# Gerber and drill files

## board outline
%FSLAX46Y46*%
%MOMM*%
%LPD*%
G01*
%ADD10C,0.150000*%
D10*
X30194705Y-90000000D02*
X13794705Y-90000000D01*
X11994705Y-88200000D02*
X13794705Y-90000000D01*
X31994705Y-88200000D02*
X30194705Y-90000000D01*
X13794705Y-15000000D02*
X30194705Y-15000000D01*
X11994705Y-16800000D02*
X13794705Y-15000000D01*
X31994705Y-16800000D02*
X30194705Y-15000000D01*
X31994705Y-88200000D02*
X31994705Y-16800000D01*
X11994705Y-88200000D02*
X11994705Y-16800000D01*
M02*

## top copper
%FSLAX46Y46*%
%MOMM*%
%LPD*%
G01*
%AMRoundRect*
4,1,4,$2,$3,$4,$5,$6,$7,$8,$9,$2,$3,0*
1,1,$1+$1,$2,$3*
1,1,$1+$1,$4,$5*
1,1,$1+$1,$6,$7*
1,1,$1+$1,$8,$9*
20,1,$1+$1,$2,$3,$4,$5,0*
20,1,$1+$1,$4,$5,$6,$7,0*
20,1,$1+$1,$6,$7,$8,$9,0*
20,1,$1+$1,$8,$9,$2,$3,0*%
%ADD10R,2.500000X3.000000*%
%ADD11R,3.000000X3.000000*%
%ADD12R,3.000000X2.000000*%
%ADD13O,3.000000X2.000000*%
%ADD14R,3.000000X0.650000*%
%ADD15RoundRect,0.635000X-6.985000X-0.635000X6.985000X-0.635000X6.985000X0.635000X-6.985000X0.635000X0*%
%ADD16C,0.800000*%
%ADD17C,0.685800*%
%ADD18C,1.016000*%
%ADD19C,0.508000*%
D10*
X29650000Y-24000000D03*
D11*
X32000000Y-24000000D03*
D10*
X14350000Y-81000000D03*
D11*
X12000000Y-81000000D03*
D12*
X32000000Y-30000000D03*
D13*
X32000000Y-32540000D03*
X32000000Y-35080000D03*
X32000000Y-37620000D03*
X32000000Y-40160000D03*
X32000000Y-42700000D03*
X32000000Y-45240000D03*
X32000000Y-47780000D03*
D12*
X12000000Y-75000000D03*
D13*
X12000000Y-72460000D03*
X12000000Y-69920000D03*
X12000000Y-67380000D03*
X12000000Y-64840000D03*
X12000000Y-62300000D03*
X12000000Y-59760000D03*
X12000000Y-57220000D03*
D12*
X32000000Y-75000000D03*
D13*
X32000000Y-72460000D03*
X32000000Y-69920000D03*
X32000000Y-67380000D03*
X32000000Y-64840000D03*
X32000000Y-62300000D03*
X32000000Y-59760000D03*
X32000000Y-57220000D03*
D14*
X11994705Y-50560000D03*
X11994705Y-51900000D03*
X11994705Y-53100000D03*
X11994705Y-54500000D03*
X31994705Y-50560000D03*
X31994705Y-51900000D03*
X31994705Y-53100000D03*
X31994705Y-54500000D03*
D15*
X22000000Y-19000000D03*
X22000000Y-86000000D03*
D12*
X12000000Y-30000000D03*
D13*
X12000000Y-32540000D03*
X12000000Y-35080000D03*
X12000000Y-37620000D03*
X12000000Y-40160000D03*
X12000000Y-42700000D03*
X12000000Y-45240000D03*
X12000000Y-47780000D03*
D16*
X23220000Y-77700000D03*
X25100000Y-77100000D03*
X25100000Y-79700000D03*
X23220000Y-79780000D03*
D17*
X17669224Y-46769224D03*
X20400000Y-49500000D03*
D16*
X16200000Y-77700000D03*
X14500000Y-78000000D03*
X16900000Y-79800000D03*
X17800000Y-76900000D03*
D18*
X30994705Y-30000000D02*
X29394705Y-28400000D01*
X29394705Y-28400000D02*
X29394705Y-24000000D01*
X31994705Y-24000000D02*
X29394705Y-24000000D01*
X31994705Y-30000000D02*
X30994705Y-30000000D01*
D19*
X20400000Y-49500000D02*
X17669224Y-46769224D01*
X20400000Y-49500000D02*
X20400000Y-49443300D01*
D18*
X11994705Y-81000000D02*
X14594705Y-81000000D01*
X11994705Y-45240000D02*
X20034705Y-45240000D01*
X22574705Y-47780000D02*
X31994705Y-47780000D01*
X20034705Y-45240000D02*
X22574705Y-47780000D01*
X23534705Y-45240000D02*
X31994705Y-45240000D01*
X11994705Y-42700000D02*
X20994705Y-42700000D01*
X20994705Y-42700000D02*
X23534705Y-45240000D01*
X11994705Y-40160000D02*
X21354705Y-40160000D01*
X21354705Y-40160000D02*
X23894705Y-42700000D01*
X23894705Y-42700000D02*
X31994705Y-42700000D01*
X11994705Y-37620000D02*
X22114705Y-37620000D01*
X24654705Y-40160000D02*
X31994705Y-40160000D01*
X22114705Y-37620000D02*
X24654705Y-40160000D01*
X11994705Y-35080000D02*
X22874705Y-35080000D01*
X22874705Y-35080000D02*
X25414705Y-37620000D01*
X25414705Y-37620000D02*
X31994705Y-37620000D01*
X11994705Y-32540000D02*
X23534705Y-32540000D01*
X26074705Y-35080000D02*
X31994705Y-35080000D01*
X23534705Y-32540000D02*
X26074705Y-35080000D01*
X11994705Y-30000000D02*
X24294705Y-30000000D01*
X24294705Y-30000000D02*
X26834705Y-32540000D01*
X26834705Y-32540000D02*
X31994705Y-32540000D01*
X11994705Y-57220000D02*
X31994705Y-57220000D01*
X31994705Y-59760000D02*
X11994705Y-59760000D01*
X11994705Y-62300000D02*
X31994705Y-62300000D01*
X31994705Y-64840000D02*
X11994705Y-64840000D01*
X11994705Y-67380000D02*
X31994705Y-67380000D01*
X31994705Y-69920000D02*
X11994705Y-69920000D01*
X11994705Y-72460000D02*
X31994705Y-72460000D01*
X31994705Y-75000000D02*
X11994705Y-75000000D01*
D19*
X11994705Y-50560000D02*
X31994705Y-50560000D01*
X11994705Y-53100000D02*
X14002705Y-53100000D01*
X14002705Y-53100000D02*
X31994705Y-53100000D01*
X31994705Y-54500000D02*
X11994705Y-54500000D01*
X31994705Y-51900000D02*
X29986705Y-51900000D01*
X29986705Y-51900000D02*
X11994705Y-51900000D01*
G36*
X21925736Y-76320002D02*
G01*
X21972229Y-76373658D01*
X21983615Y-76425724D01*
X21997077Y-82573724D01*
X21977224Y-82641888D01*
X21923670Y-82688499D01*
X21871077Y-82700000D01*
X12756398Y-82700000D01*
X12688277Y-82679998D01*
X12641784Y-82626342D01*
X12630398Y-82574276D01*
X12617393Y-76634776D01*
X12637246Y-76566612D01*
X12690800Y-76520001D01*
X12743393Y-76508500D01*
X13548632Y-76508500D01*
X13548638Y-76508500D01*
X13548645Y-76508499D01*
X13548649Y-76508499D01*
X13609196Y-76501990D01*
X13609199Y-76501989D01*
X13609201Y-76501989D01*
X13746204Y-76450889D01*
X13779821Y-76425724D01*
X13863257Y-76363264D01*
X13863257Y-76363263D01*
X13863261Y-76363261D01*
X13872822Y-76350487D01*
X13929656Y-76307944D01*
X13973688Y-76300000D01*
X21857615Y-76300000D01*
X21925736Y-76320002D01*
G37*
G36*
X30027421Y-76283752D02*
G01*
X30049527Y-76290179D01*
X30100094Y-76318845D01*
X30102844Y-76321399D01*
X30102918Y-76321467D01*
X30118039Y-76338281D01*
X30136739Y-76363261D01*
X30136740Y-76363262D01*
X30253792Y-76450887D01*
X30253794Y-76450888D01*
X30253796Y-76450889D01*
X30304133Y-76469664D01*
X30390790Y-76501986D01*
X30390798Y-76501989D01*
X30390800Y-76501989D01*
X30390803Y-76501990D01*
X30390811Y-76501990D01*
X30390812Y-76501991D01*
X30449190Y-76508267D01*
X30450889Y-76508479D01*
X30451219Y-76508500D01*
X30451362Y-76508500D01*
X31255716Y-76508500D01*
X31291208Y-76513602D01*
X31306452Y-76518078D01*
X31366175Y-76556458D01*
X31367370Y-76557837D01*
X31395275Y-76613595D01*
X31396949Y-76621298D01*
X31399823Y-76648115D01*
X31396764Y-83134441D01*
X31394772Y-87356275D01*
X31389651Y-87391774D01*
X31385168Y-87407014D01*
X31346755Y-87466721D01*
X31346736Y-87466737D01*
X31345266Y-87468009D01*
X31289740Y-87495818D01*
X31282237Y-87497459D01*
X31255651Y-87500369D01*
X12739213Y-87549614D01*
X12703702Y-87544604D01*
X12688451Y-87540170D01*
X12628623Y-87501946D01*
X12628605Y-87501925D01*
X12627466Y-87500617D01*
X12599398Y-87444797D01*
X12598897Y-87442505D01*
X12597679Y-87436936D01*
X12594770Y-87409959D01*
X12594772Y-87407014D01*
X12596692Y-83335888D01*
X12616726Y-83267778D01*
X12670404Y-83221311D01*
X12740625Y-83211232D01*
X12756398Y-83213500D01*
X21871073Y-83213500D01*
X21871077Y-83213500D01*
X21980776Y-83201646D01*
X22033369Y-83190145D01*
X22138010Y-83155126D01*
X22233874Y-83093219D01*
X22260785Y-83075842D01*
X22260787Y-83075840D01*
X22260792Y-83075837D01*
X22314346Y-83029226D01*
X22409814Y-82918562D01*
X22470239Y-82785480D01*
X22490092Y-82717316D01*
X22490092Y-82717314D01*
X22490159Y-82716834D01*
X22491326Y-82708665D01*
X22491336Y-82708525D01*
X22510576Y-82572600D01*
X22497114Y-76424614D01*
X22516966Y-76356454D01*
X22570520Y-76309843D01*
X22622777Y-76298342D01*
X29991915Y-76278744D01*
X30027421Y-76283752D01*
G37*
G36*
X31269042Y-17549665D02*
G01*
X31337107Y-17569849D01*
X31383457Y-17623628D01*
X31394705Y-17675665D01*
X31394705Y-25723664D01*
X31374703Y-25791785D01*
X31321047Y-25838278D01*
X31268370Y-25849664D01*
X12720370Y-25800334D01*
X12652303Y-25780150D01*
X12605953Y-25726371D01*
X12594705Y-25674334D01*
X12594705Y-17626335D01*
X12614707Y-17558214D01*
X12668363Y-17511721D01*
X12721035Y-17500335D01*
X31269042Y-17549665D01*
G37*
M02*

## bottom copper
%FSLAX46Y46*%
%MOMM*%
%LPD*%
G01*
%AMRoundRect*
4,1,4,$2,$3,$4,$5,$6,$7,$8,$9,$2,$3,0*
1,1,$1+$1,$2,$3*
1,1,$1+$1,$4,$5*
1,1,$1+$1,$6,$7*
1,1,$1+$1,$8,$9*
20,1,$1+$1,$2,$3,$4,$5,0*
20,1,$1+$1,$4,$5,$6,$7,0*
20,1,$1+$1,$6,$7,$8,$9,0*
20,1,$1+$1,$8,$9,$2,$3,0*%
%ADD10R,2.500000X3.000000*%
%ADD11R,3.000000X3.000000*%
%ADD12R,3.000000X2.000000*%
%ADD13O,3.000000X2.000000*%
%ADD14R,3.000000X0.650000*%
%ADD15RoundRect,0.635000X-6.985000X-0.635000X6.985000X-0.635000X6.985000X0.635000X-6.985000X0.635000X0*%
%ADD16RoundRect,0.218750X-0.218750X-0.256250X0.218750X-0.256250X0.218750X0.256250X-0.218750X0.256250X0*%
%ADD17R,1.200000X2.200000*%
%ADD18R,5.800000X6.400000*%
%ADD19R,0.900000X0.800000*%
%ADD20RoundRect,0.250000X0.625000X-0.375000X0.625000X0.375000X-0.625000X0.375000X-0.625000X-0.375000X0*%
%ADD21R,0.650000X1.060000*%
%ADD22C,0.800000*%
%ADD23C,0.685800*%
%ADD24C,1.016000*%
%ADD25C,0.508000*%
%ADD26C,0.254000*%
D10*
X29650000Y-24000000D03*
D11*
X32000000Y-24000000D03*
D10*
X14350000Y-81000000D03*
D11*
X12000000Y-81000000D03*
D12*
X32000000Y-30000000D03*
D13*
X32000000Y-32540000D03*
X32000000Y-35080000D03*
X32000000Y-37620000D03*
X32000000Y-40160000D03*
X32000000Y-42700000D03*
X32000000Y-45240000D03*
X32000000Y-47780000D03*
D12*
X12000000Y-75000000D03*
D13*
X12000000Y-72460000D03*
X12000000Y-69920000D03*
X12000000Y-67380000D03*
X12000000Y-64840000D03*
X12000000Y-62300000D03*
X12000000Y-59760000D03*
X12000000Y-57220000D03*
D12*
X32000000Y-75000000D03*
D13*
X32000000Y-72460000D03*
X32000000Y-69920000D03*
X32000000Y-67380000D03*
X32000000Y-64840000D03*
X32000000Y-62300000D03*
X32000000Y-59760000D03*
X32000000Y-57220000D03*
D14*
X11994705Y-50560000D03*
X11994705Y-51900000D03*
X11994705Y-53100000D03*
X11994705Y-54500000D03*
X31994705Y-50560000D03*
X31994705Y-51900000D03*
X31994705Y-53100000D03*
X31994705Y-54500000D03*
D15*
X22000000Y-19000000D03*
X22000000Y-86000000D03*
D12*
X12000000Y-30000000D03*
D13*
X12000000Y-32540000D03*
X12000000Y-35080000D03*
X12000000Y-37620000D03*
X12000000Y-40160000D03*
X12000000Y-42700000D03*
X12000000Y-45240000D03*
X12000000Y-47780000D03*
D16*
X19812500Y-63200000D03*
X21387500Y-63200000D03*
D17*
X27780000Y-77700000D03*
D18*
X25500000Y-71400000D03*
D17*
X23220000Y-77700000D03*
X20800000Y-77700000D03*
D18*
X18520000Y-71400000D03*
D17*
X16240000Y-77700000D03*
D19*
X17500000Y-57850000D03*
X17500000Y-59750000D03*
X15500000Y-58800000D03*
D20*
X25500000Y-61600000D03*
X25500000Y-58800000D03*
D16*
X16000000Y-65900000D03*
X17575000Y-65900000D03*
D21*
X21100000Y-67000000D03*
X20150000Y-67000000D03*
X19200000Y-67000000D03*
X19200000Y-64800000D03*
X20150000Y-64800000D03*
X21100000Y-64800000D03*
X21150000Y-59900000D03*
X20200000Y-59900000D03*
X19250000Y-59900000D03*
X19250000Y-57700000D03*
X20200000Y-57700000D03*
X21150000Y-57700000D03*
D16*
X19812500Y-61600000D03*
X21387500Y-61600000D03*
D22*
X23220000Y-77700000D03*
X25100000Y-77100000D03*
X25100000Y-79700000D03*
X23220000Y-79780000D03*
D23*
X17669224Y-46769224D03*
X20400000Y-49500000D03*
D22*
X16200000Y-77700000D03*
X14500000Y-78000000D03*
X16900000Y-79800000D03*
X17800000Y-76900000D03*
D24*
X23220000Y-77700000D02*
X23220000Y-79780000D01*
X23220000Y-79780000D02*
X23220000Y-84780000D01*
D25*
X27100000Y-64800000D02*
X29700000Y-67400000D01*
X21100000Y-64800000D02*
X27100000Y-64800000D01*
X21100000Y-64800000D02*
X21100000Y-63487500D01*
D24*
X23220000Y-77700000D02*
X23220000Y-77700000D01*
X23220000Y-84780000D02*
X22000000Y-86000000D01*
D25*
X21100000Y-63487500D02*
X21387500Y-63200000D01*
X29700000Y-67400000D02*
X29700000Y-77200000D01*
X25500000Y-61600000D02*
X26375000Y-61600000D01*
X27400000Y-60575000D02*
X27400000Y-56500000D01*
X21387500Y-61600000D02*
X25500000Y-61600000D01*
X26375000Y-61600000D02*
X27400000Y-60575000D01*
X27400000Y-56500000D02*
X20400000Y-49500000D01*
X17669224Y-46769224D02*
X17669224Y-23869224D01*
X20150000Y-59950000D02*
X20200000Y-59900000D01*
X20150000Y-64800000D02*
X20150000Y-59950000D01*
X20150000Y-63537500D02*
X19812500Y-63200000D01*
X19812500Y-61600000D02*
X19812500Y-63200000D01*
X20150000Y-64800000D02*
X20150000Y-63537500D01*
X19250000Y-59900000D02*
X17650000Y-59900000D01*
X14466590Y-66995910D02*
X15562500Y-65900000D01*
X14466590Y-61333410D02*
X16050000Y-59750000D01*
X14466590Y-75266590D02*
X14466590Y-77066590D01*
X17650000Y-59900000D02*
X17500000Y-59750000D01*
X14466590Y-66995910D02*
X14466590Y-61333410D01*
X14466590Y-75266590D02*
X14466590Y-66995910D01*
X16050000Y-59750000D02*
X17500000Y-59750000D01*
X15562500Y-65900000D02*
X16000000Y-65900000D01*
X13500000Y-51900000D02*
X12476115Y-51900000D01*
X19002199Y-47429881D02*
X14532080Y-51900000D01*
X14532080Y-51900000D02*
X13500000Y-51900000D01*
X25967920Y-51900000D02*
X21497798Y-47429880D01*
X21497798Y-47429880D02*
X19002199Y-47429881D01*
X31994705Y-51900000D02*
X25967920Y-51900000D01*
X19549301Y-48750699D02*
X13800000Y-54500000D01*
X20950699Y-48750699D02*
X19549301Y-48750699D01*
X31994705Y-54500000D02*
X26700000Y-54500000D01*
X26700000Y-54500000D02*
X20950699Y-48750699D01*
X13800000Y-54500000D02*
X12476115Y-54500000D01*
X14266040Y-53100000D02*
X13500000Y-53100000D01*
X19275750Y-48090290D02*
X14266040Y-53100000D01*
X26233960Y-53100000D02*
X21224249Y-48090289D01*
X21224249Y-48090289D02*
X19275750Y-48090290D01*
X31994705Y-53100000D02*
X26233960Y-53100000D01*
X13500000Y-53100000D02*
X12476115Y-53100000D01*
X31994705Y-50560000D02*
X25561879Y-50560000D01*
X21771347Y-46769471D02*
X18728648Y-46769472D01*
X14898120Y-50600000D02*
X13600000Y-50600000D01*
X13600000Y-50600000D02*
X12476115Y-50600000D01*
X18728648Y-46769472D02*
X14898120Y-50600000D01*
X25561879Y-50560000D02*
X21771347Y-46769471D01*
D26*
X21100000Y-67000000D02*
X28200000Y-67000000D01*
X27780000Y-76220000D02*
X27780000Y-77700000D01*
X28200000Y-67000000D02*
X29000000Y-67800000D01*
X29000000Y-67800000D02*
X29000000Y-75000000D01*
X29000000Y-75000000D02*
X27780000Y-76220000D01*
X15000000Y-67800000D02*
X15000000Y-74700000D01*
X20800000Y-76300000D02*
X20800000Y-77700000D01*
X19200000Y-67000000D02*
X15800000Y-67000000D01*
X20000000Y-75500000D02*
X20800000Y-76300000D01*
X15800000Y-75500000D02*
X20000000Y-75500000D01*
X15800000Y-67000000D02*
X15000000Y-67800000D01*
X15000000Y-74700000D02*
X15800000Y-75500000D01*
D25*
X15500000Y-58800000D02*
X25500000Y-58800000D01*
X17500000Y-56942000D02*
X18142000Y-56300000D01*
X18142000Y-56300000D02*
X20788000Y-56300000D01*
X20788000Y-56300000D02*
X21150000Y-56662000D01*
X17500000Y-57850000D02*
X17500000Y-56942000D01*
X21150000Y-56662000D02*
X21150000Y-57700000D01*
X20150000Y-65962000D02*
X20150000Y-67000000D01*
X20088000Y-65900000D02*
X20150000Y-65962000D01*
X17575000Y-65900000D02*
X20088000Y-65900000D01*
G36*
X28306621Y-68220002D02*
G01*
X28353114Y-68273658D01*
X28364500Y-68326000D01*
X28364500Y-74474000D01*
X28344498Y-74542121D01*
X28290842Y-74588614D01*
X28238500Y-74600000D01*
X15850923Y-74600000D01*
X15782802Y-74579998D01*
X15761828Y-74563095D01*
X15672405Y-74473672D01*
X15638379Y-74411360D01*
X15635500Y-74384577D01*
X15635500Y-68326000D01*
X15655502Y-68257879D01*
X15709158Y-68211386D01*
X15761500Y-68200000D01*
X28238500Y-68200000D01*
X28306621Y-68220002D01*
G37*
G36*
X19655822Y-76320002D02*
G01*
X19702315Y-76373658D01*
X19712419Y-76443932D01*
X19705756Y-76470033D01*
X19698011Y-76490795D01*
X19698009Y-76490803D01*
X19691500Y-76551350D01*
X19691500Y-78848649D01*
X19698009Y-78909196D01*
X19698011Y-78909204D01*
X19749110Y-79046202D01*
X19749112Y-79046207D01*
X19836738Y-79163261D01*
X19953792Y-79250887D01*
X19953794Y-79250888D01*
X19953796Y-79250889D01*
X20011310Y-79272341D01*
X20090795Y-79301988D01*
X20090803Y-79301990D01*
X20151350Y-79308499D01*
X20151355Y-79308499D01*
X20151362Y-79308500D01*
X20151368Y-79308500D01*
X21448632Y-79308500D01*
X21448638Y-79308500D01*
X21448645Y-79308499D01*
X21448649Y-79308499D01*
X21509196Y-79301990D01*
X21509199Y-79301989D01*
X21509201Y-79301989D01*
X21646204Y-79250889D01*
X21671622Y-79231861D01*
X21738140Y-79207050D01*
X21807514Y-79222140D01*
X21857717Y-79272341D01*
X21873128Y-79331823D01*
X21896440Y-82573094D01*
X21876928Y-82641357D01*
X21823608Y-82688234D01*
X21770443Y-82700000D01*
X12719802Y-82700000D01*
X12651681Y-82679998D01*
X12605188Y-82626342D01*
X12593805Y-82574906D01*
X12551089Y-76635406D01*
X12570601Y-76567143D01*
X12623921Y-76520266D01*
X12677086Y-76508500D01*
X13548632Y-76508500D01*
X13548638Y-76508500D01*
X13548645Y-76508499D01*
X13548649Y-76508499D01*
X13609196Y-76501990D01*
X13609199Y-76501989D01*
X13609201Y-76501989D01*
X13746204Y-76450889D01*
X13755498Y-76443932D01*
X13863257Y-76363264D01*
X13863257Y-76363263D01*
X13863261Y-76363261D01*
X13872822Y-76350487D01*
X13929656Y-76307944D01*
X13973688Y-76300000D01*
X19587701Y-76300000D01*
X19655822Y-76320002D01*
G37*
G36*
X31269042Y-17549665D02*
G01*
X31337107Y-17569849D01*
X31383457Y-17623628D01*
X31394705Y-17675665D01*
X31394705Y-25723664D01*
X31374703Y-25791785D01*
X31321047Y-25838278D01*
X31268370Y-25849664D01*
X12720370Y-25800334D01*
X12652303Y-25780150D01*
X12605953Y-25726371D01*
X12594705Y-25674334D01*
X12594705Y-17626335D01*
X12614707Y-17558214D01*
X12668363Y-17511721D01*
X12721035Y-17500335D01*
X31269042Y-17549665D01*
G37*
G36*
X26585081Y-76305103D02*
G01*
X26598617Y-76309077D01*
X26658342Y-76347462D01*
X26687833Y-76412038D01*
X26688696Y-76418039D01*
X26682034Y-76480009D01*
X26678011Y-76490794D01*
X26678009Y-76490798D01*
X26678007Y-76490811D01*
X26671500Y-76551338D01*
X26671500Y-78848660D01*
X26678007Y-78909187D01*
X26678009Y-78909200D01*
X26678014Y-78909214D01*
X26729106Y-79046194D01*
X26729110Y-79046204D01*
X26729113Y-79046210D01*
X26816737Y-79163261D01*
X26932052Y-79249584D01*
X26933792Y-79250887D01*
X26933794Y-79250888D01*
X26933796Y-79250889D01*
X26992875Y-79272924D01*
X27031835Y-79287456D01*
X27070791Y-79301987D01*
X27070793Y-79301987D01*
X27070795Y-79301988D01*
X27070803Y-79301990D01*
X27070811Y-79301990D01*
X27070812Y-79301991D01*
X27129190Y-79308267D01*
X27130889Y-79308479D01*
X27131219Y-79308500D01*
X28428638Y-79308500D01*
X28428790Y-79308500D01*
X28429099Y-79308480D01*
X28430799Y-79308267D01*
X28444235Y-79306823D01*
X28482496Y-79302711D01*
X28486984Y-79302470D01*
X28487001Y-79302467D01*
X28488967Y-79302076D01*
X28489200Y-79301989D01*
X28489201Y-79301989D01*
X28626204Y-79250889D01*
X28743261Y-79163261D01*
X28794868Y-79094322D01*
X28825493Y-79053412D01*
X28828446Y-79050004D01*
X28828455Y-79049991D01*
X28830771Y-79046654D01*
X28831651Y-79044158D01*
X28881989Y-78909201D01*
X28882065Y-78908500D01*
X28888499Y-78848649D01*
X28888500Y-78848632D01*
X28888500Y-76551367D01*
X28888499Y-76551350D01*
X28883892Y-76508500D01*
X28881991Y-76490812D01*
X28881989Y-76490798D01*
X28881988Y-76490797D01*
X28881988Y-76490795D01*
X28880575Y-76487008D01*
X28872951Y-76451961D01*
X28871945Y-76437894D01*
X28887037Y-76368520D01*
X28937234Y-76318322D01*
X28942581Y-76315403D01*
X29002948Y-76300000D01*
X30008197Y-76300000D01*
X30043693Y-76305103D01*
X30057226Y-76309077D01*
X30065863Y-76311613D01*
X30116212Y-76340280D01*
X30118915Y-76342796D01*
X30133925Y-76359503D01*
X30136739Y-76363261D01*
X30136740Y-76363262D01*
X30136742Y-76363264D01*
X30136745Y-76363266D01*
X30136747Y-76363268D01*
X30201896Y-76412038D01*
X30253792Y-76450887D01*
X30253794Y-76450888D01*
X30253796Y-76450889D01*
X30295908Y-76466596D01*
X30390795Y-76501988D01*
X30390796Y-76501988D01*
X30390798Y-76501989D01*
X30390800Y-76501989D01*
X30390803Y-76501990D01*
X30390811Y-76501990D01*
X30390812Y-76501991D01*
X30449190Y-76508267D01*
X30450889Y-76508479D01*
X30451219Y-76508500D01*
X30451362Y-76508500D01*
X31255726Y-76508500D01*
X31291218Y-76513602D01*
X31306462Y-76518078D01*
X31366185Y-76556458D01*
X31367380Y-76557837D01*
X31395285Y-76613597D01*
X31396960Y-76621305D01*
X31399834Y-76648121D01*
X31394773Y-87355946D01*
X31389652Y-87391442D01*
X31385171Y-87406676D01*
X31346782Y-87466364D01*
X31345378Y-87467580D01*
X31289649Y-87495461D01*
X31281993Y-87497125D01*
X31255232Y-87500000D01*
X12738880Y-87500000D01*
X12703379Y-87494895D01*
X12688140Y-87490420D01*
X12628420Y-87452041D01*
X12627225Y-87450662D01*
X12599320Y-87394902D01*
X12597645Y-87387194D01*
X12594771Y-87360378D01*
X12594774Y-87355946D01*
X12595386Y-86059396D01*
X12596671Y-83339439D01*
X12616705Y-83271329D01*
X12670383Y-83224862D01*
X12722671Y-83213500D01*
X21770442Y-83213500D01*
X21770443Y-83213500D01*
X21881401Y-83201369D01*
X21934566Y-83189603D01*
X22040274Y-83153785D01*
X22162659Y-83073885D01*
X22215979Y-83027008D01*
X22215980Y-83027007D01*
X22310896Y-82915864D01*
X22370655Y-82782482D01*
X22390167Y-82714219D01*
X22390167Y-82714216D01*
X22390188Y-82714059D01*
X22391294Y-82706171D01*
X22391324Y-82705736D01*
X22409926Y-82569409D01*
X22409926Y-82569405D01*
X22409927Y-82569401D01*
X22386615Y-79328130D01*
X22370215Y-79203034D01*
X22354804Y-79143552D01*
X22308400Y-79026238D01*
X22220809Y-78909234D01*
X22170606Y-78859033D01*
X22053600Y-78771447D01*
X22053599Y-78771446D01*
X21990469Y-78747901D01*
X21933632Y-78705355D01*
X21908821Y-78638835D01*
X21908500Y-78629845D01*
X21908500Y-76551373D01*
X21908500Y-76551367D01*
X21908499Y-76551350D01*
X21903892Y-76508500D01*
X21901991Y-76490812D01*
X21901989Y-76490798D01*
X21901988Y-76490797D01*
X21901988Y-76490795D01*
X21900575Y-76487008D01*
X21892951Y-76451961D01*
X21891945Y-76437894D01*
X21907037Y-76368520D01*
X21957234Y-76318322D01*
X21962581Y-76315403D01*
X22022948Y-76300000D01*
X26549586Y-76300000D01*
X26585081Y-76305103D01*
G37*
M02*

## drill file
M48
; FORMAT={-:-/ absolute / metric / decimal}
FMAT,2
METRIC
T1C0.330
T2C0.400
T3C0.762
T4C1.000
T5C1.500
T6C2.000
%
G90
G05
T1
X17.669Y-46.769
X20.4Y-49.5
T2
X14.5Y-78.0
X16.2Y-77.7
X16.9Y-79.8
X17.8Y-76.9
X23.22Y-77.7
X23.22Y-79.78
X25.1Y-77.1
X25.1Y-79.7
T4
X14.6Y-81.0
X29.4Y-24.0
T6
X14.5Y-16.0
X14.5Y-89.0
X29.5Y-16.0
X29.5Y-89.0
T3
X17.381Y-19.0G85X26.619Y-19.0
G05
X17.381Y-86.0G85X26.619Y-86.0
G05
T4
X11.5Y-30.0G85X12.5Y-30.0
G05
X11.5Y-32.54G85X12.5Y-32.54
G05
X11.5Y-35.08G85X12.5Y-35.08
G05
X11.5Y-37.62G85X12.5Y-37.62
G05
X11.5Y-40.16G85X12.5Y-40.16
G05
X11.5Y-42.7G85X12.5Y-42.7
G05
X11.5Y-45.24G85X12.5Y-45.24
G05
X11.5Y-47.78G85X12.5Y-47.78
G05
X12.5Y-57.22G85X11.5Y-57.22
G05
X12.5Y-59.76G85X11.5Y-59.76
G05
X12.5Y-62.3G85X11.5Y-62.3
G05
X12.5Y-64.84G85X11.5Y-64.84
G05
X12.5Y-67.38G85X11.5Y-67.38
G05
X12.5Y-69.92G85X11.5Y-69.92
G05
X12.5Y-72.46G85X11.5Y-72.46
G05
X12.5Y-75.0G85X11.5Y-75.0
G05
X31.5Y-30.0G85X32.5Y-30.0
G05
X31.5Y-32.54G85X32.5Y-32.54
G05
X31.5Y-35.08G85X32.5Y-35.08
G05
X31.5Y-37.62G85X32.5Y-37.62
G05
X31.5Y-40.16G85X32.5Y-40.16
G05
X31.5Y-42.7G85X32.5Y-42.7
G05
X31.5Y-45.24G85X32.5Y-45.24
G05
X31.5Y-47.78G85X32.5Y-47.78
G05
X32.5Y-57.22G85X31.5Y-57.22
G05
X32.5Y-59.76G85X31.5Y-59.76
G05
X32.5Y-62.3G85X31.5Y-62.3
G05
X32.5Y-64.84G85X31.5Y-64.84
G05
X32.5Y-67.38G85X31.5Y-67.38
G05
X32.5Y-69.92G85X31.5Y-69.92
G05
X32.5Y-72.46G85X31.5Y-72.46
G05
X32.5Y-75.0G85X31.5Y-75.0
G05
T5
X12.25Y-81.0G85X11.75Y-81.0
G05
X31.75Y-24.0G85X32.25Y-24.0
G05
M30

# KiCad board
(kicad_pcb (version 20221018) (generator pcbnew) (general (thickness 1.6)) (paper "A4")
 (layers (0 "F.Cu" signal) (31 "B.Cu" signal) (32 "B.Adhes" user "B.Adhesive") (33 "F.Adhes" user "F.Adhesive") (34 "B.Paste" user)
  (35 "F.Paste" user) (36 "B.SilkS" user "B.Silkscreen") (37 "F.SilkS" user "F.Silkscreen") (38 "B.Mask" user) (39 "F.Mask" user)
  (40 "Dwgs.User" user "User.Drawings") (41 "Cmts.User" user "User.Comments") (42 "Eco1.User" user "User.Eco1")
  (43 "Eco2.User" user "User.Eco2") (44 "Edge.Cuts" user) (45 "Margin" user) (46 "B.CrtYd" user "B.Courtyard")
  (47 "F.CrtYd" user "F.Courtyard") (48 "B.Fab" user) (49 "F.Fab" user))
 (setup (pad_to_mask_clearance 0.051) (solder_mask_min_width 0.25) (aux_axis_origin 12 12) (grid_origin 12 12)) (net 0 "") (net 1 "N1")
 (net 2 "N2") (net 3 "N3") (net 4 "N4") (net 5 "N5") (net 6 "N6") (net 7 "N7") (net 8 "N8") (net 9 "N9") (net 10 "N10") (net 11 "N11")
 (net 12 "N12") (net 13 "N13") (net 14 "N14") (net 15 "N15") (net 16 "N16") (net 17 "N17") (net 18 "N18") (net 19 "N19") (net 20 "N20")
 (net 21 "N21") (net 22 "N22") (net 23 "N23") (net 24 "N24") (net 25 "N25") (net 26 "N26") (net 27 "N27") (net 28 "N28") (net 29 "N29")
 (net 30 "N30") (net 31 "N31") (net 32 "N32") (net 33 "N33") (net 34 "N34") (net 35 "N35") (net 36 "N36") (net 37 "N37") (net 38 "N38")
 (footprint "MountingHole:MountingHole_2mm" (layer "F.Cu") (at 14.5 16)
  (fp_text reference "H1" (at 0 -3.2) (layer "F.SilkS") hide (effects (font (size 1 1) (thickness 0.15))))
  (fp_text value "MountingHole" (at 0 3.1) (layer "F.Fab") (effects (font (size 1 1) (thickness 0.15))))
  (pad "" np_thru_hole circle (at 0 0) (size 2 2) (drill 2) (layers "*.Cu" "*.Mask")))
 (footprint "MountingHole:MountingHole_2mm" (layer "F.Cu") (at 29.5 16)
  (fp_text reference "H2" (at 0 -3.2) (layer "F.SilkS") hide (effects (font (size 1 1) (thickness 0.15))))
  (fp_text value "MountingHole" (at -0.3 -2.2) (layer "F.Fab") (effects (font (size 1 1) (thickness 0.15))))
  (pad "" np_thru_hole circle (at 0 0) (size 2 2) (drill 2) (layers "*.Cu" "*.Mask")))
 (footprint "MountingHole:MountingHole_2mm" (layer "F.Cu") (at 29.5 89)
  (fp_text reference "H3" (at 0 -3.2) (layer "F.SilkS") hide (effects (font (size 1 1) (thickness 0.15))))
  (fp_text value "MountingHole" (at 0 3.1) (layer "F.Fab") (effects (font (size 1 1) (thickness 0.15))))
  (pad "" np_thru_hole circle (at 0 0) (size 2 2) (drill 2) (layers "*.Cu" "*.Mask")))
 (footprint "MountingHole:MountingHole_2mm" (layer "F.Cu") (at 14.5 89)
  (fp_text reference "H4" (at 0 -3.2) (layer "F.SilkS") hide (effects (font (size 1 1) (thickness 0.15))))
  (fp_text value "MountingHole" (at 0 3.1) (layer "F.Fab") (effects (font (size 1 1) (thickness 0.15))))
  (pad "" np_thru_hole circle (at 0 0) (size 2 2) (drill 2) (layers "*.Cu" "*.Mask")))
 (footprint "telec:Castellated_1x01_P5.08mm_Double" (layer "F.Cu") (at 32 24)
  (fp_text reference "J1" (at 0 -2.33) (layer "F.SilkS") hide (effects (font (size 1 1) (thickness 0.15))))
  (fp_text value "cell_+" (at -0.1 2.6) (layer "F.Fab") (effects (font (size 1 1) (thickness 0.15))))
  (pad "1" thru_hole rect (at -2.6 0) (size 2.5 3) (drill 1 (offset 0.25 0)) (layers "*.Cu" "*.Mask") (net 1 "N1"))
  (pad "1" thru_hole rect (at 0 0) (size 3 3) (drill oval 2 1.5) (layers "*.Cu" "*.Mask") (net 1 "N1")))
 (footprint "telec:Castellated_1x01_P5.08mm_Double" (layer "F.Cu") (at 12 81 180)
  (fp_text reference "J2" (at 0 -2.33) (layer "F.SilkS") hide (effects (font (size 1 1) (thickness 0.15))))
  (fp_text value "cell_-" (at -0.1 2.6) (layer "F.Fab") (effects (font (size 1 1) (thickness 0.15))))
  (pad "1" thru_hole rect (at -2.6 0 180) (size 2.5 3) (drill 1 (offset 0.25 0)) (layers "*.Cu" "*.Mask") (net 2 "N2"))
  (pad "1" thru_hole rect (at 0 0 180) (size 3 3) (drill oval 2 1.5) (layers "*.Cu" "*.Mask") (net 2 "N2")))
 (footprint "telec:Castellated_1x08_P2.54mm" (layer "F.Cu") (at 32 30)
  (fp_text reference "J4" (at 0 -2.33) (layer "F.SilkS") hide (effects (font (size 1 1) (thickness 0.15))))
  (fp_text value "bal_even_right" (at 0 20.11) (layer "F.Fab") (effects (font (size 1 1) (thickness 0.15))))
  (pad "1" thru_hole rect (at 0 0) (size 3 2) (drill oval 2 1) (layers "*.Cu" "*.Mask") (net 1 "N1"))
  (pad "2" thru_hole oval (at 0 2.54) (size 3 2) (drill oval 2 1) (layers "*.Cu" "*.Mask") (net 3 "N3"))
  (pad "3" thru_hole oval (at 0 5.08) (size 3 2) (drill oval 2 1) (layers "*.Cu" "*.Mask") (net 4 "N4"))
  (pad "4" thru_hole oval (at 0 7.62) (size 3 2) (drill oval 2 1) (layers "*.Cu" "*.Mask") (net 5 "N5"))
  (pad "5" thru_hole oval (at 0 10.16) (size 3 2) (drill oval 2 1) (layers "*.Cu" "*.Mask") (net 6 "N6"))
  (pad "6" thru_hole oval (at 0 12.7) (size 3 2) (drill oval 2 1) (layers "*.Cu" "*.Mask") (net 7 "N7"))
  (pad "7" thru_hole oval (at 0 15.24) (size 3 2) (drill oval 2 1) (layers "*.Cu" "*.Mask") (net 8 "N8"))
  (pad "8" thru_hole oval (at 0 17.78) (size 3 2) (drill oval 2 1) (layers "*.Cu" "*.Mask") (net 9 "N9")))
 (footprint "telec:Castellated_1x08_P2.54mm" (layer "F.Cu") (at 12 75 180)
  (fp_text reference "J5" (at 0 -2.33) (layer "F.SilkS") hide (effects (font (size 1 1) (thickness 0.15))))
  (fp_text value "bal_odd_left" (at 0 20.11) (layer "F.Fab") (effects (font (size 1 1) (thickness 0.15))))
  (pad "1" thru_hole rect (at 0 0 180) (size 3 2) (drill oval 2 1) (layers "*.Cu" "*.Mask") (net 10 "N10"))
  (pad "2" thru_hole oval (at 0 2.54 180) (size 3 2) (drill oval 2 1) (layers "*.Cu" "*.Mask") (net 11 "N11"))
  (pad "3" thru_hole oval (at 0 5.08 180) (size 3 2) (drill oval 2 1) (layers "*.Cu" "*.Mask") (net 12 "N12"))
  (pad "4" thru_hole oval (at 0 7.62 180) (size 3 2) (drill oval 2 1) (layers "*.Cu" "*.Mask") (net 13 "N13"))
  (pad "5" thru_hole oval (at 0 10.16 180) (size 3 2) (drill oval 2 1) (layers "*.Cu" "*.Mask") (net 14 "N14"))
  (pad "6" thru_hole oval (at 0 12.7 180) (size 3 2) (drill oval 2 1) (layers "*.Cu" "*.Mask") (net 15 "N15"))
  (pad "7" thru_hole oval (at 0 15.24 180) (size 3 2) (drill oval 2 1) (layers "*.Cu" "*.Mask") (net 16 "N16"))
  (pad "8" thru_hole oval (at 0 17.78 180) (size 3 2) (drill oval 2 1) (layers "*.Cu" "*.Mask") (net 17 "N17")))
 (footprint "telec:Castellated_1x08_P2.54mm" (layer "F.Cu") (at 32 75 180)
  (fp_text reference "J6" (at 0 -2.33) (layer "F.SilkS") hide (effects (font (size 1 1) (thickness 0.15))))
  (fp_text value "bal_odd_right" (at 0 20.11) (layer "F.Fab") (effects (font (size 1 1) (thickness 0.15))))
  (pad "1" thru_hole rect (at 0 0 180) (size 3 2) (drill oval 2 1) (layers "*.Cu" "*.Mask") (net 10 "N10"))
  (pad "2" thru_hole oval (at 0 2.54 180) (size 3 2) (drill oval 2 1) (layers "*.Cu" "*.Mask") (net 11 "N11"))
  (pad "3" thru_hole oval (at 0 5.08 180) (size 3 2) (drill oval 2 1) (layers "*.Cu" "*.Mask") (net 12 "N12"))
  (pad "4" thru_hole oval (at 0 7.62 180) (size 3 2) (drill oval 2 1) (layers "*.Cu" "*.Mask") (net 13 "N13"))
  (pad "5" thru_hole oval (at 0 10.16 180) (size 3 2) (drill oval 2 1) (layers "*.Cu" "*.Mask") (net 14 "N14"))
  (pad "6" thru_hole oval (at 0 12.7 180) (size 3 2) (drill oval 2 1) (layers "*.Cu" "*.Mask") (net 15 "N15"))
  (pad "7" thru_hole oval (at 0 15.24 180) (size 3 2) (drill oval 2 1) (layers "*.Cu" "*.Mask") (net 16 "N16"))
  (pad "8" thru_hole oval (at 0 17.78 180) (size 3 2) (drill oval 2 1) (layers "*.Cu" "*.Mask") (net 17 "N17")))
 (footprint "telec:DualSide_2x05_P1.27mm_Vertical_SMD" (layer "F.Cu") (at 11.994705 52.6)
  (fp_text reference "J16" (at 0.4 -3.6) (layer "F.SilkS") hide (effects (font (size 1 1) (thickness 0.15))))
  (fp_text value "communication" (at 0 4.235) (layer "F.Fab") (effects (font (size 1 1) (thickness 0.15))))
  (pad "1" smd rect (at 0 -2.04) (size 3 0.65) (layers "*.Mask" "F.Cu") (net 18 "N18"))
  (pad "2" smd rect (at 0 -2.04) (size 3 0.65) (layers "*.Mask" "B.Cu") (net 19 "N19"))
  (pad "3" smd rect (at 0 -0.7) (size 3 0.65) (layers "*.Mask" "F.Cu") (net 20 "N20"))
  (pad "4" smd rect (at 0 -0.7) (size 3 0.65) (layers "*.Mask" "B.Cu") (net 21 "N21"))
  (pad "5" smd rect (at 0 0.5) (size 3 0.65) (layers "*.Mask" "F.Cu") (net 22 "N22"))
  (pad "6" smd rect (at 0 0.5) (size 3 0.65) (layers "*.Mask" "B.Cu") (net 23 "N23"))
  (pad "7" smd rect (at 0 1.9) (size 3 0.65) (layers "*.Mask" "F.Cu") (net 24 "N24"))
  (pad "8" smd rect (at 0 1.9) (size 3 0.65) (layers "*.Mask" "B.Cu") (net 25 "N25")))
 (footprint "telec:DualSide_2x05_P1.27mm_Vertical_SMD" (layer "F.Cu") (at 31.994705 52.6)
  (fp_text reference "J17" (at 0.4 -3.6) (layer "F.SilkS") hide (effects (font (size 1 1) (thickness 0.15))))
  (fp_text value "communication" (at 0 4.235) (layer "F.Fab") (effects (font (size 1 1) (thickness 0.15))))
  (pad "1" smd rect (at 0 -2.04) (size 3 0.65) (layers "*.Mask" "F.Cu") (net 18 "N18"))
  (pad "2" smd rect (at 0 -2.04) (size 3 0.65) (layers "*.Mask" "B.Cu") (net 19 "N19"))
  (pad "3" smd rect (at 0 -0.7) (size 3 0.65) (layers "*.Mask" "F.Cu") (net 20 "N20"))
  (pad "4" smd rect (at 0 -0.7) (size 3 0.65) (layers "*.Mask" "B.Cu") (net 21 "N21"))
  (pad "5" smd rect (at 0 0.5) (size 3 0.65) (layers "*.Mask" "F.Cu") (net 22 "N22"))
  (pad "6" smd rect (at 0 0.5) (size 3 0.65) (layers "*.Mask" "B.Cu") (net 23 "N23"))
  (pad "7" smd rect (at 0 1.9) (size 3 0.65) (layers "*.Mask" "F.Cu") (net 24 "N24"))
  (pad "8" smd rect (at 0 1.9) (size 3 0.65) (layers "*.Mask" "B.Cu") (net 25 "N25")))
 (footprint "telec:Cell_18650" (layer "F.Cu") (at 22 19)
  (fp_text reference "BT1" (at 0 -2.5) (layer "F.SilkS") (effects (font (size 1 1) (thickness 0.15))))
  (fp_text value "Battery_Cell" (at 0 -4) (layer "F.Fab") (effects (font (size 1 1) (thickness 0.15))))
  (pad "1" thru_hole roundrect (at 0 0) (size 15.24 2.54) (drill oval 10 0.762) (layers "*.Cu" "*.Mask") (roundrect_rratio 0.25)
   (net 1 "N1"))
  (pad "2" thru_hole roundrect (at 0 67) (size 15.24 2.54) (drill oval 10 0.762) (layers "*.Cu" "*.Mask") (roundrect_rratio 0.25)
   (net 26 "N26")))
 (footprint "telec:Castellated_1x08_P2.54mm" (layer "F.Cu") (at 12 30)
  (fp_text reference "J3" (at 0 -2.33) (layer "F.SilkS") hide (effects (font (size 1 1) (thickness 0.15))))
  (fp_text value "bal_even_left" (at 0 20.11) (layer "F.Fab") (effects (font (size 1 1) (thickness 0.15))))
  (pad "1" thru_hole rect (at 0 0) (size 3 2) (drill oval 2 1) (layers "*.Cu" "*.Mask") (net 3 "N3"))
  (pad "2" thru_hole oval (at 0 2.54) (size 3 2) (drill oval 2 1) (layers "*.Cu" "*.Mask") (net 4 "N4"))
  (pad "3" thru_hole oval (at 0 5.08) (size 3 2) (drill oval 2 1) (layers "*.Cu" "*.Mask") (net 5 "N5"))
  (pad "4" thru_hole oval (at 0 7.62) (size 3 2) (drill oval 2 1) (layers "*.Cu" "*.Mask") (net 6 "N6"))
  (pad "5" thru_hole oval (at 0 10.16) (size 3 2) (drill oval 2 1) (layers "*.Cu" "*.Mask") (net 7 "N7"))
  (pad "6" thru_hole oval (at 0 12.7) (size 3 2) (drill oval 2 1) (layers "*.Cu" "*.Mask") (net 8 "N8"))
  (pad "7" thru_hole oval (at 0 15.24) (size 3 2) (drill oval 2 1) (layers "*.Cu" "*.Mask") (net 9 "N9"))
  (pad "8" thru_hole oval (at 0 17.78) (size 3 2) (drill oval 2 1) (layers "*.Cu" "*.Mask") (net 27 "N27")))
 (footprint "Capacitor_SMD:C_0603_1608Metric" (layer "B.Cu") (at 20.6 63.2)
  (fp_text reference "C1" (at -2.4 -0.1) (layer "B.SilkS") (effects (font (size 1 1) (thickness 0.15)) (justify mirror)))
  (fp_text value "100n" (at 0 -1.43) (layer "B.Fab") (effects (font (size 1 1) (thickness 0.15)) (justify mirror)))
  (pad "1" smd roundrect (at -0.7875 0) (size 0.875 0.95) (layers "B.Cu" "B.Paste" "B.Mask") (roundrect_rratio 0.25) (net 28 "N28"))
  (pad "2" smd roundrect (at 0.7875 0) (size 0.875 0.95) (layers "B.Cu" "B.Paste" "B.Mask") (roundrect_rratio 0.25) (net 26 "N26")))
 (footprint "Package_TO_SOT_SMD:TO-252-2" (layer "B.Cu") (at 25.5 73.5 90)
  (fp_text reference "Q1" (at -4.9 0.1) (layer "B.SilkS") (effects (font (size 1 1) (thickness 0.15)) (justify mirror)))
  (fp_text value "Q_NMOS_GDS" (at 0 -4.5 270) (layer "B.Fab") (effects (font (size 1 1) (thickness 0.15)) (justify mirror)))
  (pad "" smd rect (at 0.425 -1.525 90) (size 3.05 2.75) (layers "B.Paste"))
  (pad "" smd rect (at 0.425 1.525 90) (size 3.05 2.75) (layers "B.Paste"))
  (pad "" smd rect (at 3.775 -1.525 90) (size 3.05 2.75) (layers "B.Paste"))
  (pad "" smd rect (at 3.775 1.525 90) (size 3.05 2.75) (layers "B.Paste"))
  (pad "1" smd rect (at -4.2 2.28 90) (size 2.2 1.2) (layers "B.Cu" "B.Paste" "B.Mask") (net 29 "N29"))
  (pad "2" smd rect (at 2.1 0 90) (size 6.4 5.8) (layers "B.Cu" "B.Mask") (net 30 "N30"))
  (pad "3" smd rect (at -4.2 -2.28 90) (size 2.2 1.2) (layers "B.Cu" "B.Paste" "B.Mask") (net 26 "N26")))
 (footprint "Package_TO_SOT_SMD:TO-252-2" (layer "B.Cu") (at 18.52 73.5 90)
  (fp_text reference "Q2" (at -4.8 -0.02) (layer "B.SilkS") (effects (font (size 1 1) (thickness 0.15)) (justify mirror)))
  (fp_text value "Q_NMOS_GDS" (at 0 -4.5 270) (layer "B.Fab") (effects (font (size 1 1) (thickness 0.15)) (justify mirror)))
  (pad "" smd rect (at 0.425 -1.525 90) (size 3.05 2.75) (layers "B.Paste"))
  (pad "" smd rect (at 0.425 1.525 90) (size 3.05 2.75) (layers "B.Paste"))
  (pad "" smd rect (at 3.775 -1.525 90) (size 3.05 2.75) (layers "B.Paste"))
  (pad "" smd rect (at 3.775 1.525 90) (size 3.05 2.75) (layers "B.Paste"))
  (pad "1" smd rect (at -4.2 2.28 90) (size 2.2 1.2) (layers "B.Cu" "B.Paste" "B.Mask") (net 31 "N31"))
  (pad "2" smd rect (at 2.1 0 90) (size 6.4 5.8) (layers "B.Cu" "B.Mask") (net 30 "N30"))
  (pad "3" smd rect (at -4.2 -2.28 90) (size 2.2 1.2) (layers "B.Cu" "B.Paste" "B.Mask") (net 2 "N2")))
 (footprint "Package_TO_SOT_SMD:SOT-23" (layer "B.Cu") (at 16.5 58.8 180)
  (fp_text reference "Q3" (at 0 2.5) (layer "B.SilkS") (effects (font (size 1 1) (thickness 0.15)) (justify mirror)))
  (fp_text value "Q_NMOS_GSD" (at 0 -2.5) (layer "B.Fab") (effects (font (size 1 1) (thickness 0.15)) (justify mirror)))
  (pad "1" smd rect (at -1 0.95 180) (size 0.9 0.8) (layers "B.Cu" "B.Paste" "B.Mask") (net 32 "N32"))
  (pad "2" smd rect (at -1 -0.95 180) (size 0.9 0.8) (layers "B.Cu" "B.Paste" "B.Mask") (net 2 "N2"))
  (pad "3" smd rect (at 1 0 180) (size 0.9 0.8) (layers "B.Cu" "B.Paste" "B.Mask") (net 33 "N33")))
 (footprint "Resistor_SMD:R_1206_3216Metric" (layer "B.Cu") (at 25.5 60.2 90)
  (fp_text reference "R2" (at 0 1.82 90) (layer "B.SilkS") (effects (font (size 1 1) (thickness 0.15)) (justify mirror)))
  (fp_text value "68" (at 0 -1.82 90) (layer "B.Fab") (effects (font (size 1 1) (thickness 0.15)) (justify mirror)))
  (pad "1" smd roundrect (at -1.4 0 90) (size 1.25 1.75) (layers "B.Cu" "B.Paste" "B.Mask") (roundrect_rratio 0.2) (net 1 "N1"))
  (pad "2" smd roundrect (at 1.4 0 90) (size 1.25 1.75) (layers "B.Cu" "B.Paste" "B.Mask") (roundrect_rratio 0.2) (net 33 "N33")))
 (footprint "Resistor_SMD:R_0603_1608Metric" (layer "B.Cu") (at 16.7875 65.9)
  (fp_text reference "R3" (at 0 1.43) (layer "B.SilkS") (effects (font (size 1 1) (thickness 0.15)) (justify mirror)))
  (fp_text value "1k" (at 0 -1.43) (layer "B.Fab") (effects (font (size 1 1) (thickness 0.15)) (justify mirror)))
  (pad "1" smd roundrect (at -0.7875 0) (size 0.875 0.95) (layers "B.Cu" "B.Paste" "B.Mask") (roundrect_rratio 0.25) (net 2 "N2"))
  (pad "2" smd roundrect (at 0.7875 0) (size 0.875 0.95) (layers "B.Cu" "B.Paste" "B.Mask") (roundrect_rratio 0.25) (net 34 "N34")))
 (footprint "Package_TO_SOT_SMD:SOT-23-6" (layer "B.Cu") (at 20.15 65.9 90)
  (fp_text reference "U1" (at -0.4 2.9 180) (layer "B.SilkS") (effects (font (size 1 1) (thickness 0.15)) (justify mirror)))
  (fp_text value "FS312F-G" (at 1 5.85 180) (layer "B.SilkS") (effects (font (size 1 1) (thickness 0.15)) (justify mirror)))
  (pad "1" smd rect (at -1.1 0.95 90) (size 1.06 0.65) (layers "B.Cu" "B.Paste" "B.Mask") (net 29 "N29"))
  (pad "2" smd rect (at -1.1 0 90) (size 1.06 0.65) (layers "B.Cu" "B.Paste" "B.Mask") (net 34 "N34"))
  (pad "3" smd rect (at -1.1 -0.95 90) (size 1.06 0.65) (layers "B.Cu" "B.Paste" "B.Mask") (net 31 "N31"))
  (pad "4" smd rect (at 1.1 -0.95 90) (size 1.06 0.65) (layers "B.Cu" "B.Paste" "B.Mask") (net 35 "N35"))
  (pad "5" smd rect (at 1.1 0 90) (size 1.06 0.65) (layers "B.Cu" "B.Paste" "B.Mask") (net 28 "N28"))
  (pad "6" smd rect (at 1.1 0.95 90) (size 1.06 0.65) (layers "B.Cu" "B.Paste" "B.Mask") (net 26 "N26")))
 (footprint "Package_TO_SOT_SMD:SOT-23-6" (layer "B.Cu") (at 20.2 58.8 90)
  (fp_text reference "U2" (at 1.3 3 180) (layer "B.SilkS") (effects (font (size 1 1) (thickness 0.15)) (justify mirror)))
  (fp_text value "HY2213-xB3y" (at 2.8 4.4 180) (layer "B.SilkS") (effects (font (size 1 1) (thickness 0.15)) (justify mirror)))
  (pad "1" smd rect (at -1.1 0.95 90) (size 1.06 0.65) (layers "B.Cu" "B.Paste" "B.Mask") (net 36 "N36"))
  (pad "2" smd rect (at -1.1 0 90) (size 1.06 0.65) (layers "B.Cu" "B.Paste" "B.Mask") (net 28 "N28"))
  (pad "3" smd rect (at -1.1 -0.95 90) (size 1.06 0.65) (layers "B.Cu" "B.Paste" "B.Mask") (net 2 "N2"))
  (pad "4" smd rect (at 1.1 -0.95 90) (size 1.06 0.65) (layers "B.Cu" "B.Paste" "B.Mask") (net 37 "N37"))
  (pad "5" smd rect (at 1.1 0 90) (size 1.06 0.65) (layers "B.Cu" "B.Paste" "B.Mask") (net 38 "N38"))
  (pad "6" smd rect (at 1.1 0.95 90) (size 1.06 0.65) (layers "B.Cu" "B.Paste" "B.Mask") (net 32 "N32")))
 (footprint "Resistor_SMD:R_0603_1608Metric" (layer "B.Cu") (at 20.6 61.6)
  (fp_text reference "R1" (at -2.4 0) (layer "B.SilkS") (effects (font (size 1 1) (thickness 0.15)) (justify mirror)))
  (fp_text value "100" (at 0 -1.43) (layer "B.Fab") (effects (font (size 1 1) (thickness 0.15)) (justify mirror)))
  (pad "1" smd roundrect (at -0.7875 0) (size 0.875 0.95) (layers "B.Cu" "B.Paste" "B.Mask") (roundrect_rratio 0.25) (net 28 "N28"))
  (pad "2" smd roundrect (at 0.7875 0) (size 0.875 0.95) (layers "B.Cu" "B.Paste" "B.Mask") (roundrect_rratio 0.25) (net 1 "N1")))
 (gr_line (start 30.194705 90) (end 13.794705 90) (stroke (width 0.15) (type solid)) (layer "Edge.Cuts"))
 (gr_line (start 11.994705 88.2) (end 13.794705 90) (stroke (width 0.15) (type solid)) (layer "Edge.Cuts"))
 (gr_line (start 31.994705 88.2) (end 30.194705 90) (stroke (width 0.15) (type solid)) (layer "Edge.Cuts"))
 (gr_line (start 13.794705 15) (end 30.194705 15) (stroke (width 0.15) (type solid)) (layer "Edge.Cuts"))
 (gr_line (start 11.994705 16.8) (end 13.794705 15) (stroke (width 0.15) (type solid)) (layer "Edge.Cuts"))
 (gr_line (start 31.994705 16.8) (end 30.194705 15) (stroke (width 0.15) (type solid)) (layer "Edge.Cuts"))
 (gr_line (start 31.994705 88.2) (end 31.994705 16.8) (stroke (width 0.15) (type solid)) (layer "Edge.Cuts"))
 (gr_line (start 11.994705 88.2) (end 11.994705 16.8) (stroke (width 0.15) (type solid)) (layer "Edge.Cuts"))
 (via (at 23.22 77.7) (size 0.8) (drill 0.4) (layers "F.Cu" "B.Cu") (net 26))
 (via (at 25.1 77.1) (size 0.8) (drill 0.4) (layers "F.Cu" "B.Cu") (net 26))
 (via (at 25.1 79.7) (size 0.8) (drill 0.4) (layers "F.Cu" "B.Cu") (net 26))
 (via (at 23.22 79.78) (size 0.8) (drill 0.4) (layers "F.Cu" "B.Cu") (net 26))
 (segment (start 23.22 77.7) (end 23.22 79.78) (width 1.016) (layer "B.Cu") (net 26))
 (segment (start 23.22 79.78) (end 23.22 84.78) (width 1.016) (layer "B.Cu") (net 26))
 (segment (start 27.1 64.8) (end 29.7 67.4) (width 0.508) (layer "B.Cu") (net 26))
 (segment (start 21.1 64.8) (end 27.1 64.8) (width 0.508) (layer "B.Cu") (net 26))
 (segment (start 21.1 64.8) (end 21.1 63.4875) (width 0.508) (layer "B.Cu") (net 26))
 (segment (start 23.22 77.7) (end 23.22 77.7) (width 1.016) (layer "B.Cu") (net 26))
 (segment (start 23.22 84.78) (end 22 86) (width 1.016) (layer "B.Cu") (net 26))
 (segment (start 21.1 63.4875) (end 21.3875 63.2) (width 0.508) (layer "B.Cu") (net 26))
 (segment (start 29.7 67.4) (end 29.7 77.2) (width 0.508) (layer "B.Cu") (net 26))
 (segment (start 30.994705 30) (end 29.394705 28.4) (width 1.016) (layer "F.Cu") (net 1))
 (segment (start 29.394705 28.4) (end 29.394705 24) (width 1.016) (layer "F.Cu") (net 1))
 (segment (start 31.994705 24) (end 29.394705 24) (width 1.016) (layer "F.Cu") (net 1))
 (segment (start 31.994705 30) (end 30.994705 30) (width 1.016) (layer "F.Cu") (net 1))
 (segment (start 20.4 49.5) (end 17.669224 46.769224) (width 0.508) (layer "F.Cu") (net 1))
 (segment (start 20.4 49.5) (end 20.4 49.4433) (width 0.508) (layer "F.Cu") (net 1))
 (via (at 17.669224 46.769224) (size 0.6858) (drill 0.3302) (layers "F.Cu" "B.Cu") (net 1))
 (via (at 20.4 49.5) (size 0.6858) (drill 0.3302) (layers "F.Cu" "B.Cu") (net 1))
 (segment (start 25.5 61.6) (end 26.375 61.6) (width 0.508) (layer "B.Cu") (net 1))
 (segment (start 27.4 60.575) (end 27.4 56.5) (width 0.508) (layer "B.Cu") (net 1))
 (segment (start 21.3875 61.6) (end 25.5 61.6) (width 0.508) (layer "B.Cu") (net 1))
 (segment (start 26.375 61.6) (end 27.4 60.575) (width 0.508) (layer "B.Cu") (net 1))
 (segment (start 27.4 56.5) (end 20.4 49.5) (width 0.508) (layer "B.Cu") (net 1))
 (segment (start 17.669224 46.769224) (end 17.669224 23.869224) (width 0.508) (layer "B.Cu") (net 1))
 (segment (start 20.15 59.95) (end 20.2 59.9) (width 0.508) (layer "B.Cu") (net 28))
 (segment (start 20.15 64.8) (end 20.15 59.95) (width 0.508) (layer "B.Cu") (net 28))
 (segment (start 20.15 63.5375) (end 19.8125 63.2) (width 0.508) (layer "B.Cu") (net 28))
 (segment (start 19.8125 61.6) (end 19.8125 63.2) (width 0.508) (layer "B.Cu") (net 28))
 (segment (start 20.15 64.8) (end 20.15 63.5375) (width 0.508) (layer "B.Cu") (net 28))
 (segment (start 11.994705 81) (end 14.594705 81) (width 1.016) (layer "F.Cu") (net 2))
 (via (at 16.2 77.7) (size 0.8) (drill 0.4) (layers "F.Cu" "B.Cu") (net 2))
 (via (at 14.5 78) (size 0.8) (drill 0.4) (layers "F.Cu" "B.Cu") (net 2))
 (via (at 16.9 79.8) (size 0.8) (drill 0.4) (layers "F.Cu" "B.Cu") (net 2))
 (via (at 17.8 76.9) (size 0.8) (drill 0.4) (layers "F.Cu" "B.Cu") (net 2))
 (segment (start 19.25 59.9) (end 17.65 59.9) (width 0.508) (layer "B.Cu") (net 2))
 (segment (start 14.46659 66.99591) (end 15.5625 65.9) (width 0.508) (layer "B.Cu") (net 2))
 (segment (start 14.46659 61.33341) (end 16.05 59.75) (width 0.508) (layer "B.Cu") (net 2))
 (segment (start 14.46659 75.26659) (end 14.46659 77.06659) (width 0.508) (layer "B.Cu") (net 2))
 (segment (start 17.65 59.9) (end 17.5 59.75) (width 0.508) (layer "B.Cu") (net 2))
 (segment (start 14.46659 66.99591) (end 14.46659 61.33341) (width 0.508) (layer "B.Cu") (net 2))
 (segment (start 14.46659 75.26659) (end 14.46659 66.99591) (width 0.508) (layer "B.Cu") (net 2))
 (segment (start 16.05 59.75) (end 17.5 59.75) (width 0.508) (layer "B.Cu") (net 2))
 (segment (start 15.5625 65.9) (end 16 65.9) (width 0.508) (layer "B.Cu") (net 2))
 (segment (start 11.994705 45.24) (end 20.034705 45.24) (width 1.016) (layer "F.Cu") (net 9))
 (segment (start 22.574705 47.78) (end 31.994705 47.78) (width 1.016) (layer "F.Cu") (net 9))
 (segment (start 20.034705 45.24) (end 22.574705 47.78) (width 1.016) (layer "F.Cu") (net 9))
 (segment (start 23.534705 45.24) (end 31.994705 45.24) (width 1.016) (layer "F.Cu") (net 8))
 (segment (start 11.994705 42.7) (end 20.994705 42.7) (width 1.016) (layer "F.Cu") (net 8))
 (segment (start 20.994705 42.7) (end 23.534705 45.24) (width 1.016) (layer "F.Cu") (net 8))
 (segment (start 11.994705 40.16) (end 21.354705 40.16) (width 1.016) (layer "F.Cu") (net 7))
 (segment (start 21.354705 40.16) (end 23.894705 42.7) (width 1.016) (layer "F.Cu") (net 7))
 (segment (start 23.894705 42.7) (end 31.994705 42.7) (width 1.016) (layer "F.Cu") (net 7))
 (segment (start 11.994705 37.62) (end 22.114705 37.62) (width 1.016) (layer "F.Cu") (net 6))
 (segment (start 24.654705 40.16) (end 31.994705 40.16) (width 1.016) (layer "F.Cu") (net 6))
 (segment (start 22.114705 37.62) (end 24.654705 40.16) (width 1.016) (layer "F.Cu") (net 6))
 (segment (start 11.994705 35.08) (end 22.874705 35.08) (width 1.016) (layer "F.Cu") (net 5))
 (segment (start 22.874705 35.08) (end 25.414705 37.62) (width 1.016) (layer "F.Cu") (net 5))
 (segment (start 25.414705 37.62) (end 31.994705 37.62) (width 1.016) (layer "F.Cu") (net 5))
 (segment (start 11.994705 32.54) (end 23.534705 32.54) (width 1.016) (layer "F.Cu") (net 4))
 (segment (start 26.074705 35.08) (end 31.994705 35.08) (width 1.016) (layer "F.Cu") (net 4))
 (segment (start 23.534705 32.54) (end 26.074705 35.08) (width 1.016) (layer "F.Cu") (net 4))
 (segment (start 11.994705 30) (end 24.294705 30) (width 1.016) (layer "F.Cu") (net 3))
 (segment (start 24.294705 30) (end 26.834705 32.54) (width 1.016) (layer "F.Cu") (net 3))
 (segment (start 26.834705 32.54) (end 31.994705 32.54) (width 1.016) (layer "F.Cu") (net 3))
 (segment (start 11.994705 57.22) (end 31.994705 57.22) (width 1.016) (layer "F.Cu") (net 17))
 (segment (start 31.994705 59.76) (end 11.994705 59.76) (width 1.016) (layer "F.Cu") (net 16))
 (segment (start 11.994705 62.3) (end 31.994705 62.3) (width 1.016) (layer "F.Cu") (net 15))
 (segment (start 31.994705 64.84) (end 11.994705 64.84) (width 1.016) (layer "F.Cu") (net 14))
 (segment (start 11.994705 67.38) (end 31.994705 67.38) (width 1.016) (layer "F.Cu") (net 13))
 (segment (start 31.994705 69.92) (end 11.994705 69.92) (width 1.016) (layer "F.Cu") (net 12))
 (segment (start 11.994705 72.46) (end 31.994705 72.46) (width 1.016) (layer "F.Cu") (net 11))
 (segment (start 31.994705 75) (end 11.994705 75) (width 1.016) (layer "F.Cu") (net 10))
 (segment (start 13.5 51.9) (end 12.476115 51.9) (width 0.508) (layer "B.Cu") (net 21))
 (segment (start 19.002199 47.429881) (end 14.53208 51.9) (width 0.508) (layer "B.Cu") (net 21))
 (segment (start 14.53208 51.9) (end 13.5 51.9) (width 0.508) (layer "B.Cu") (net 21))
 (segment (start 25.96792 51.9) (end 21.497798 47.42988) (width 0.508) (layer "B.Cu") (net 21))
 (segment (start 21.497798 47.42988) (end 19.002199 47.429881) (width 0.508) (layer "B.Cu") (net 21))
 (segment (start 31.994705 51.9) (end 25.96792 51.9) (width 0.508) (layer "B.Cu") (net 21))
 (segment (start 19.549301 48.750699) (end 13.8 54.5) (width 0.508) (layer "B.Cu") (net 25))
 (segment (start 20.950699 48.750699) (end 19.549301 48.750699) (width 0.508) (layer "B.Cu") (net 25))
 (segment (start 31.994705 54.5) (end 26.7 54.5) (width 0.508) (layer "B.Cu") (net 25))
 (segment (start 26.7 54.5) (end 20.950699 48.750699) (width 0.508) (layer "B.Cu") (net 25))
 (segment (start 13.8 54.5) (end 12.476115 54.5) (width 0.508) (layer "B.Cu") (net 25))
 (segment (start 11.994705 50.56) (end 31.994705 50.56) (width 0.508) (layer "F.Cu") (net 18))
 (segment (start 14.26604 53.1) (end 13.5 53.1) (width 0.508) (layer "B.Cu") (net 23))
 (segment (start 19.27575 48.09029) (end 14.26604 53.1) (width 0.508) (layer "B.Cu") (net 23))
 (segment (start 26.23396 53.1) (end 21.224249 48.090289) (width 0.508) (layer "B.Cu") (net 23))
 (segment (start 21.224249 48.090289) (end 19.27575 48.09029) (width 0.508) (layer "B.Cu") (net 23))
 (segment (start 31.994705 53.1) (end 26.23396 53.1) (width 0.508) (layer "B.Cu") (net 23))
 (segment (start 13.5 53.1) (end 12.476115 53.1) (width 0.508) (layer "B.Cu") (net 23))
 (segment (start 11.994705 53.1) (end 14.002705 53.1) (width 0.508) (layer "F.Cu") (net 22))
 (segment (start 14.002705 53.1) (end 31.994705 53.1) (width 0.508) (layer "F.Cu") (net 22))
 (segment (start 31.994705 54.5) (end 11.994705 54.5) (width 0.508) (layer "F.Cu") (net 24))
 (segment (start 31.994705 51.9) (end 29.986705 51.9) (width 0.508) (layer "F.Cu") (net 20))
 (segment (start 29.986705 51.9) (end 11.994705 51.9) (width 0.508) (layer "F.Cu") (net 20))
 (segment (start 31.994705 50.56) (end 25.561879 50.56) (width 0.508) (layer "B.Cu") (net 19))
 (segment (start 21.771347 46.769471) (end 18.728648 46.769472) (width 0.508) (layer "B.Cu") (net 19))
 (segment (start 14.89812 50.6) (end 13.6 50.6) (width 0.508) (layer "B.Cu") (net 19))
 (segment (start 13.6 50.6) (end 12.476115 50.6) (width 0.508) (layer "B.Cu") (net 19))
 (segment (start 18.728648 46.769472) (end 14.89812 50.6) (width 0.508) (layer "B.Cu") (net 19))
 (segment (start 25.561879 50.56) (end 21.771347 46.769471) (width 0.508) (layer "B.Cu") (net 19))
 (segment (start 21.1 67) (end 28.2 67) (width 0.254) (layer "B.Cu") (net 29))
 (segment (start 27.78 76.22) (end 27.78 77.7) (width 0.254) (layer "B.Cu") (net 29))
 (segment (start 28.2 67) (end 29 67.8) (width 0.254) (layer "B.Cu") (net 29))
 (segment (start 29 67.8) (end 29 75) (width 0.254) (layer "B.Cu") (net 29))
 (segment (start 29 75) (end 27.78 76.22) (width 0.254) (layer "B.Cu") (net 29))
 (segment (start 15 67.8) (end 15 74.7) (width 0.254) (layer "B.Cu") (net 31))
 (segment (start 20.8 76.3) (end 20.8 77.7) (width 0.254) (layer "B.Cu") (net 31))
 (segment (start 19.2 67) (end 15.8 67) (width 0.254) (layer "B.Cu") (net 31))
 (segment (start 20 75.5) (end 20.8 76.3) (width 0.254) (layer "B.Cu") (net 31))
 (segment (start 15.8 75.5) (end 20 75.5) (width 0.254) (layer "B.Cu") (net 31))
 (segment (start 15.8 67) (end 15 67.8) (width 0.254) (layer "B.Cu") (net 31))
 (segment (start 15 74.7) (end 15.8 75.5) (width 0.254) (layer "B.Cu") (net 31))
 (segment (start 15.5 58.8) (end 25.5 58.8) (width 0.508) (layer "B.Cu") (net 33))
 (segment (start 17.5 56.942) (end 18.142 56.3) (width 0.508) (layer "B.Cu") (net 32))
 (segment (start 18.142 56.3) (end 20.788 56.3) (width 0.508) (layer "B.Cu") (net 32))
 (segment (start 20.788 56.3) (end 21.15 56.662) (width 0.508) (layer "B.Cu") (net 32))
 (segment (start 17.5 57.85) (end 17.5 56.942) (width 0.508) (layer "B.Cu") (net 32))
 (segment (start 21.15 56.662) (end 21.15 57.7) (width 0.508) (layer "B.Cu") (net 32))
 (segment (start 20.15 65.962) (end 20.15 67) (width 0.508) (layer "B.Cu") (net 34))
 (segment (start 20.088 65.9) (end 20.15 65.962) (width 0.508) (layer "B.Cu") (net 34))
 (segment (start 17.575 65.9) (end 20.088 65.9) (width 0.508) (layer "B.Cu") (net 34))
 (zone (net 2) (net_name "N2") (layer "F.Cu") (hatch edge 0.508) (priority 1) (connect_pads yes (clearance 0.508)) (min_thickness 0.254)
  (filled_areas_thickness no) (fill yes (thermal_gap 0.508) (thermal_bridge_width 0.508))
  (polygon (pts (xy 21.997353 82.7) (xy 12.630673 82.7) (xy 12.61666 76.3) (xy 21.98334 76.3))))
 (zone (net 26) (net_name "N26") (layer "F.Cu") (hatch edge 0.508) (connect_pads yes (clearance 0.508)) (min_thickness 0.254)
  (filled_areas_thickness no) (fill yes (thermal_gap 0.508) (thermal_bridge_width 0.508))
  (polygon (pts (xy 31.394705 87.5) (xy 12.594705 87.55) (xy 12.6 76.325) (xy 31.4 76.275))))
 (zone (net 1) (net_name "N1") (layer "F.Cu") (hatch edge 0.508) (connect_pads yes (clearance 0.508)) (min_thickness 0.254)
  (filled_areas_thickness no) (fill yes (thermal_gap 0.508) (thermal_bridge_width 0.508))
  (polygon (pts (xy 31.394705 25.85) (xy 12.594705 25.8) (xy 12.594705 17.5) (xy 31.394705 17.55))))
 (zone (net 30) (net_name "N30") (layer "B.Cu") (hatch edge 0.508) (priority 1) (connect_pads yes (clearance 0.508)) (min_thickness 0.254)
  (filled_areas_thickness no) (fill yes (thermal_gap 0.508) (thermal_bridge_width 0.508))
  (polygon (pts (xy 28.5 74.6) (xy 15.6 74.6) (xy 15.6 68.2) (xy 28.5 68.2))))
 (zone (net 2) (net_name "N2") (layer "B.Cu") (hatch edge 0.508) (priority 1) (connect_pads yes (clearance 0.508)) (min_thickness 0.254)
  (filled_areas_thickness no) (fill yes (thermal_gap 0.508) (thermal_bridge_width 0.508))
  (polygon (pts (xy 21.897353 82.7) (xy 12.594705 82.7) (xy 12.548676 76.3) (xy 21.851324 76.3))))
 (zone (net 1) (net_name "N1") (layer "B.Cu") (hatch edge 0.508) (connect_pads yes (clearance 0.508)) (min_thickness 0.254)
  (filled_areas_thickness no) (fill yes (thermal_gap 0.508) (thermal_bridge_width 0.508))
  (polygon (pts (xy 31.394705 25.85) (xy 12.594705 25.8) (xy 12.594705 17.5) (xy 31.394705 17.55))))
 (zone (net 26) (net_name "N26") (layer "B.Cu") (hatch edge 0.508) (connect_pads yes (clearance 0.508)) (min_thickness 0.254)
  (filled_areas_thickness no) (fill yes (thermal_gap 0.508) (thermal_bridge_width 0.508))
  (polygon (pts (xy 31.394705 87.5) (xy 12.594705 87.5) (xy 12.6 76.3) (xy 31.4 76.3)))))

